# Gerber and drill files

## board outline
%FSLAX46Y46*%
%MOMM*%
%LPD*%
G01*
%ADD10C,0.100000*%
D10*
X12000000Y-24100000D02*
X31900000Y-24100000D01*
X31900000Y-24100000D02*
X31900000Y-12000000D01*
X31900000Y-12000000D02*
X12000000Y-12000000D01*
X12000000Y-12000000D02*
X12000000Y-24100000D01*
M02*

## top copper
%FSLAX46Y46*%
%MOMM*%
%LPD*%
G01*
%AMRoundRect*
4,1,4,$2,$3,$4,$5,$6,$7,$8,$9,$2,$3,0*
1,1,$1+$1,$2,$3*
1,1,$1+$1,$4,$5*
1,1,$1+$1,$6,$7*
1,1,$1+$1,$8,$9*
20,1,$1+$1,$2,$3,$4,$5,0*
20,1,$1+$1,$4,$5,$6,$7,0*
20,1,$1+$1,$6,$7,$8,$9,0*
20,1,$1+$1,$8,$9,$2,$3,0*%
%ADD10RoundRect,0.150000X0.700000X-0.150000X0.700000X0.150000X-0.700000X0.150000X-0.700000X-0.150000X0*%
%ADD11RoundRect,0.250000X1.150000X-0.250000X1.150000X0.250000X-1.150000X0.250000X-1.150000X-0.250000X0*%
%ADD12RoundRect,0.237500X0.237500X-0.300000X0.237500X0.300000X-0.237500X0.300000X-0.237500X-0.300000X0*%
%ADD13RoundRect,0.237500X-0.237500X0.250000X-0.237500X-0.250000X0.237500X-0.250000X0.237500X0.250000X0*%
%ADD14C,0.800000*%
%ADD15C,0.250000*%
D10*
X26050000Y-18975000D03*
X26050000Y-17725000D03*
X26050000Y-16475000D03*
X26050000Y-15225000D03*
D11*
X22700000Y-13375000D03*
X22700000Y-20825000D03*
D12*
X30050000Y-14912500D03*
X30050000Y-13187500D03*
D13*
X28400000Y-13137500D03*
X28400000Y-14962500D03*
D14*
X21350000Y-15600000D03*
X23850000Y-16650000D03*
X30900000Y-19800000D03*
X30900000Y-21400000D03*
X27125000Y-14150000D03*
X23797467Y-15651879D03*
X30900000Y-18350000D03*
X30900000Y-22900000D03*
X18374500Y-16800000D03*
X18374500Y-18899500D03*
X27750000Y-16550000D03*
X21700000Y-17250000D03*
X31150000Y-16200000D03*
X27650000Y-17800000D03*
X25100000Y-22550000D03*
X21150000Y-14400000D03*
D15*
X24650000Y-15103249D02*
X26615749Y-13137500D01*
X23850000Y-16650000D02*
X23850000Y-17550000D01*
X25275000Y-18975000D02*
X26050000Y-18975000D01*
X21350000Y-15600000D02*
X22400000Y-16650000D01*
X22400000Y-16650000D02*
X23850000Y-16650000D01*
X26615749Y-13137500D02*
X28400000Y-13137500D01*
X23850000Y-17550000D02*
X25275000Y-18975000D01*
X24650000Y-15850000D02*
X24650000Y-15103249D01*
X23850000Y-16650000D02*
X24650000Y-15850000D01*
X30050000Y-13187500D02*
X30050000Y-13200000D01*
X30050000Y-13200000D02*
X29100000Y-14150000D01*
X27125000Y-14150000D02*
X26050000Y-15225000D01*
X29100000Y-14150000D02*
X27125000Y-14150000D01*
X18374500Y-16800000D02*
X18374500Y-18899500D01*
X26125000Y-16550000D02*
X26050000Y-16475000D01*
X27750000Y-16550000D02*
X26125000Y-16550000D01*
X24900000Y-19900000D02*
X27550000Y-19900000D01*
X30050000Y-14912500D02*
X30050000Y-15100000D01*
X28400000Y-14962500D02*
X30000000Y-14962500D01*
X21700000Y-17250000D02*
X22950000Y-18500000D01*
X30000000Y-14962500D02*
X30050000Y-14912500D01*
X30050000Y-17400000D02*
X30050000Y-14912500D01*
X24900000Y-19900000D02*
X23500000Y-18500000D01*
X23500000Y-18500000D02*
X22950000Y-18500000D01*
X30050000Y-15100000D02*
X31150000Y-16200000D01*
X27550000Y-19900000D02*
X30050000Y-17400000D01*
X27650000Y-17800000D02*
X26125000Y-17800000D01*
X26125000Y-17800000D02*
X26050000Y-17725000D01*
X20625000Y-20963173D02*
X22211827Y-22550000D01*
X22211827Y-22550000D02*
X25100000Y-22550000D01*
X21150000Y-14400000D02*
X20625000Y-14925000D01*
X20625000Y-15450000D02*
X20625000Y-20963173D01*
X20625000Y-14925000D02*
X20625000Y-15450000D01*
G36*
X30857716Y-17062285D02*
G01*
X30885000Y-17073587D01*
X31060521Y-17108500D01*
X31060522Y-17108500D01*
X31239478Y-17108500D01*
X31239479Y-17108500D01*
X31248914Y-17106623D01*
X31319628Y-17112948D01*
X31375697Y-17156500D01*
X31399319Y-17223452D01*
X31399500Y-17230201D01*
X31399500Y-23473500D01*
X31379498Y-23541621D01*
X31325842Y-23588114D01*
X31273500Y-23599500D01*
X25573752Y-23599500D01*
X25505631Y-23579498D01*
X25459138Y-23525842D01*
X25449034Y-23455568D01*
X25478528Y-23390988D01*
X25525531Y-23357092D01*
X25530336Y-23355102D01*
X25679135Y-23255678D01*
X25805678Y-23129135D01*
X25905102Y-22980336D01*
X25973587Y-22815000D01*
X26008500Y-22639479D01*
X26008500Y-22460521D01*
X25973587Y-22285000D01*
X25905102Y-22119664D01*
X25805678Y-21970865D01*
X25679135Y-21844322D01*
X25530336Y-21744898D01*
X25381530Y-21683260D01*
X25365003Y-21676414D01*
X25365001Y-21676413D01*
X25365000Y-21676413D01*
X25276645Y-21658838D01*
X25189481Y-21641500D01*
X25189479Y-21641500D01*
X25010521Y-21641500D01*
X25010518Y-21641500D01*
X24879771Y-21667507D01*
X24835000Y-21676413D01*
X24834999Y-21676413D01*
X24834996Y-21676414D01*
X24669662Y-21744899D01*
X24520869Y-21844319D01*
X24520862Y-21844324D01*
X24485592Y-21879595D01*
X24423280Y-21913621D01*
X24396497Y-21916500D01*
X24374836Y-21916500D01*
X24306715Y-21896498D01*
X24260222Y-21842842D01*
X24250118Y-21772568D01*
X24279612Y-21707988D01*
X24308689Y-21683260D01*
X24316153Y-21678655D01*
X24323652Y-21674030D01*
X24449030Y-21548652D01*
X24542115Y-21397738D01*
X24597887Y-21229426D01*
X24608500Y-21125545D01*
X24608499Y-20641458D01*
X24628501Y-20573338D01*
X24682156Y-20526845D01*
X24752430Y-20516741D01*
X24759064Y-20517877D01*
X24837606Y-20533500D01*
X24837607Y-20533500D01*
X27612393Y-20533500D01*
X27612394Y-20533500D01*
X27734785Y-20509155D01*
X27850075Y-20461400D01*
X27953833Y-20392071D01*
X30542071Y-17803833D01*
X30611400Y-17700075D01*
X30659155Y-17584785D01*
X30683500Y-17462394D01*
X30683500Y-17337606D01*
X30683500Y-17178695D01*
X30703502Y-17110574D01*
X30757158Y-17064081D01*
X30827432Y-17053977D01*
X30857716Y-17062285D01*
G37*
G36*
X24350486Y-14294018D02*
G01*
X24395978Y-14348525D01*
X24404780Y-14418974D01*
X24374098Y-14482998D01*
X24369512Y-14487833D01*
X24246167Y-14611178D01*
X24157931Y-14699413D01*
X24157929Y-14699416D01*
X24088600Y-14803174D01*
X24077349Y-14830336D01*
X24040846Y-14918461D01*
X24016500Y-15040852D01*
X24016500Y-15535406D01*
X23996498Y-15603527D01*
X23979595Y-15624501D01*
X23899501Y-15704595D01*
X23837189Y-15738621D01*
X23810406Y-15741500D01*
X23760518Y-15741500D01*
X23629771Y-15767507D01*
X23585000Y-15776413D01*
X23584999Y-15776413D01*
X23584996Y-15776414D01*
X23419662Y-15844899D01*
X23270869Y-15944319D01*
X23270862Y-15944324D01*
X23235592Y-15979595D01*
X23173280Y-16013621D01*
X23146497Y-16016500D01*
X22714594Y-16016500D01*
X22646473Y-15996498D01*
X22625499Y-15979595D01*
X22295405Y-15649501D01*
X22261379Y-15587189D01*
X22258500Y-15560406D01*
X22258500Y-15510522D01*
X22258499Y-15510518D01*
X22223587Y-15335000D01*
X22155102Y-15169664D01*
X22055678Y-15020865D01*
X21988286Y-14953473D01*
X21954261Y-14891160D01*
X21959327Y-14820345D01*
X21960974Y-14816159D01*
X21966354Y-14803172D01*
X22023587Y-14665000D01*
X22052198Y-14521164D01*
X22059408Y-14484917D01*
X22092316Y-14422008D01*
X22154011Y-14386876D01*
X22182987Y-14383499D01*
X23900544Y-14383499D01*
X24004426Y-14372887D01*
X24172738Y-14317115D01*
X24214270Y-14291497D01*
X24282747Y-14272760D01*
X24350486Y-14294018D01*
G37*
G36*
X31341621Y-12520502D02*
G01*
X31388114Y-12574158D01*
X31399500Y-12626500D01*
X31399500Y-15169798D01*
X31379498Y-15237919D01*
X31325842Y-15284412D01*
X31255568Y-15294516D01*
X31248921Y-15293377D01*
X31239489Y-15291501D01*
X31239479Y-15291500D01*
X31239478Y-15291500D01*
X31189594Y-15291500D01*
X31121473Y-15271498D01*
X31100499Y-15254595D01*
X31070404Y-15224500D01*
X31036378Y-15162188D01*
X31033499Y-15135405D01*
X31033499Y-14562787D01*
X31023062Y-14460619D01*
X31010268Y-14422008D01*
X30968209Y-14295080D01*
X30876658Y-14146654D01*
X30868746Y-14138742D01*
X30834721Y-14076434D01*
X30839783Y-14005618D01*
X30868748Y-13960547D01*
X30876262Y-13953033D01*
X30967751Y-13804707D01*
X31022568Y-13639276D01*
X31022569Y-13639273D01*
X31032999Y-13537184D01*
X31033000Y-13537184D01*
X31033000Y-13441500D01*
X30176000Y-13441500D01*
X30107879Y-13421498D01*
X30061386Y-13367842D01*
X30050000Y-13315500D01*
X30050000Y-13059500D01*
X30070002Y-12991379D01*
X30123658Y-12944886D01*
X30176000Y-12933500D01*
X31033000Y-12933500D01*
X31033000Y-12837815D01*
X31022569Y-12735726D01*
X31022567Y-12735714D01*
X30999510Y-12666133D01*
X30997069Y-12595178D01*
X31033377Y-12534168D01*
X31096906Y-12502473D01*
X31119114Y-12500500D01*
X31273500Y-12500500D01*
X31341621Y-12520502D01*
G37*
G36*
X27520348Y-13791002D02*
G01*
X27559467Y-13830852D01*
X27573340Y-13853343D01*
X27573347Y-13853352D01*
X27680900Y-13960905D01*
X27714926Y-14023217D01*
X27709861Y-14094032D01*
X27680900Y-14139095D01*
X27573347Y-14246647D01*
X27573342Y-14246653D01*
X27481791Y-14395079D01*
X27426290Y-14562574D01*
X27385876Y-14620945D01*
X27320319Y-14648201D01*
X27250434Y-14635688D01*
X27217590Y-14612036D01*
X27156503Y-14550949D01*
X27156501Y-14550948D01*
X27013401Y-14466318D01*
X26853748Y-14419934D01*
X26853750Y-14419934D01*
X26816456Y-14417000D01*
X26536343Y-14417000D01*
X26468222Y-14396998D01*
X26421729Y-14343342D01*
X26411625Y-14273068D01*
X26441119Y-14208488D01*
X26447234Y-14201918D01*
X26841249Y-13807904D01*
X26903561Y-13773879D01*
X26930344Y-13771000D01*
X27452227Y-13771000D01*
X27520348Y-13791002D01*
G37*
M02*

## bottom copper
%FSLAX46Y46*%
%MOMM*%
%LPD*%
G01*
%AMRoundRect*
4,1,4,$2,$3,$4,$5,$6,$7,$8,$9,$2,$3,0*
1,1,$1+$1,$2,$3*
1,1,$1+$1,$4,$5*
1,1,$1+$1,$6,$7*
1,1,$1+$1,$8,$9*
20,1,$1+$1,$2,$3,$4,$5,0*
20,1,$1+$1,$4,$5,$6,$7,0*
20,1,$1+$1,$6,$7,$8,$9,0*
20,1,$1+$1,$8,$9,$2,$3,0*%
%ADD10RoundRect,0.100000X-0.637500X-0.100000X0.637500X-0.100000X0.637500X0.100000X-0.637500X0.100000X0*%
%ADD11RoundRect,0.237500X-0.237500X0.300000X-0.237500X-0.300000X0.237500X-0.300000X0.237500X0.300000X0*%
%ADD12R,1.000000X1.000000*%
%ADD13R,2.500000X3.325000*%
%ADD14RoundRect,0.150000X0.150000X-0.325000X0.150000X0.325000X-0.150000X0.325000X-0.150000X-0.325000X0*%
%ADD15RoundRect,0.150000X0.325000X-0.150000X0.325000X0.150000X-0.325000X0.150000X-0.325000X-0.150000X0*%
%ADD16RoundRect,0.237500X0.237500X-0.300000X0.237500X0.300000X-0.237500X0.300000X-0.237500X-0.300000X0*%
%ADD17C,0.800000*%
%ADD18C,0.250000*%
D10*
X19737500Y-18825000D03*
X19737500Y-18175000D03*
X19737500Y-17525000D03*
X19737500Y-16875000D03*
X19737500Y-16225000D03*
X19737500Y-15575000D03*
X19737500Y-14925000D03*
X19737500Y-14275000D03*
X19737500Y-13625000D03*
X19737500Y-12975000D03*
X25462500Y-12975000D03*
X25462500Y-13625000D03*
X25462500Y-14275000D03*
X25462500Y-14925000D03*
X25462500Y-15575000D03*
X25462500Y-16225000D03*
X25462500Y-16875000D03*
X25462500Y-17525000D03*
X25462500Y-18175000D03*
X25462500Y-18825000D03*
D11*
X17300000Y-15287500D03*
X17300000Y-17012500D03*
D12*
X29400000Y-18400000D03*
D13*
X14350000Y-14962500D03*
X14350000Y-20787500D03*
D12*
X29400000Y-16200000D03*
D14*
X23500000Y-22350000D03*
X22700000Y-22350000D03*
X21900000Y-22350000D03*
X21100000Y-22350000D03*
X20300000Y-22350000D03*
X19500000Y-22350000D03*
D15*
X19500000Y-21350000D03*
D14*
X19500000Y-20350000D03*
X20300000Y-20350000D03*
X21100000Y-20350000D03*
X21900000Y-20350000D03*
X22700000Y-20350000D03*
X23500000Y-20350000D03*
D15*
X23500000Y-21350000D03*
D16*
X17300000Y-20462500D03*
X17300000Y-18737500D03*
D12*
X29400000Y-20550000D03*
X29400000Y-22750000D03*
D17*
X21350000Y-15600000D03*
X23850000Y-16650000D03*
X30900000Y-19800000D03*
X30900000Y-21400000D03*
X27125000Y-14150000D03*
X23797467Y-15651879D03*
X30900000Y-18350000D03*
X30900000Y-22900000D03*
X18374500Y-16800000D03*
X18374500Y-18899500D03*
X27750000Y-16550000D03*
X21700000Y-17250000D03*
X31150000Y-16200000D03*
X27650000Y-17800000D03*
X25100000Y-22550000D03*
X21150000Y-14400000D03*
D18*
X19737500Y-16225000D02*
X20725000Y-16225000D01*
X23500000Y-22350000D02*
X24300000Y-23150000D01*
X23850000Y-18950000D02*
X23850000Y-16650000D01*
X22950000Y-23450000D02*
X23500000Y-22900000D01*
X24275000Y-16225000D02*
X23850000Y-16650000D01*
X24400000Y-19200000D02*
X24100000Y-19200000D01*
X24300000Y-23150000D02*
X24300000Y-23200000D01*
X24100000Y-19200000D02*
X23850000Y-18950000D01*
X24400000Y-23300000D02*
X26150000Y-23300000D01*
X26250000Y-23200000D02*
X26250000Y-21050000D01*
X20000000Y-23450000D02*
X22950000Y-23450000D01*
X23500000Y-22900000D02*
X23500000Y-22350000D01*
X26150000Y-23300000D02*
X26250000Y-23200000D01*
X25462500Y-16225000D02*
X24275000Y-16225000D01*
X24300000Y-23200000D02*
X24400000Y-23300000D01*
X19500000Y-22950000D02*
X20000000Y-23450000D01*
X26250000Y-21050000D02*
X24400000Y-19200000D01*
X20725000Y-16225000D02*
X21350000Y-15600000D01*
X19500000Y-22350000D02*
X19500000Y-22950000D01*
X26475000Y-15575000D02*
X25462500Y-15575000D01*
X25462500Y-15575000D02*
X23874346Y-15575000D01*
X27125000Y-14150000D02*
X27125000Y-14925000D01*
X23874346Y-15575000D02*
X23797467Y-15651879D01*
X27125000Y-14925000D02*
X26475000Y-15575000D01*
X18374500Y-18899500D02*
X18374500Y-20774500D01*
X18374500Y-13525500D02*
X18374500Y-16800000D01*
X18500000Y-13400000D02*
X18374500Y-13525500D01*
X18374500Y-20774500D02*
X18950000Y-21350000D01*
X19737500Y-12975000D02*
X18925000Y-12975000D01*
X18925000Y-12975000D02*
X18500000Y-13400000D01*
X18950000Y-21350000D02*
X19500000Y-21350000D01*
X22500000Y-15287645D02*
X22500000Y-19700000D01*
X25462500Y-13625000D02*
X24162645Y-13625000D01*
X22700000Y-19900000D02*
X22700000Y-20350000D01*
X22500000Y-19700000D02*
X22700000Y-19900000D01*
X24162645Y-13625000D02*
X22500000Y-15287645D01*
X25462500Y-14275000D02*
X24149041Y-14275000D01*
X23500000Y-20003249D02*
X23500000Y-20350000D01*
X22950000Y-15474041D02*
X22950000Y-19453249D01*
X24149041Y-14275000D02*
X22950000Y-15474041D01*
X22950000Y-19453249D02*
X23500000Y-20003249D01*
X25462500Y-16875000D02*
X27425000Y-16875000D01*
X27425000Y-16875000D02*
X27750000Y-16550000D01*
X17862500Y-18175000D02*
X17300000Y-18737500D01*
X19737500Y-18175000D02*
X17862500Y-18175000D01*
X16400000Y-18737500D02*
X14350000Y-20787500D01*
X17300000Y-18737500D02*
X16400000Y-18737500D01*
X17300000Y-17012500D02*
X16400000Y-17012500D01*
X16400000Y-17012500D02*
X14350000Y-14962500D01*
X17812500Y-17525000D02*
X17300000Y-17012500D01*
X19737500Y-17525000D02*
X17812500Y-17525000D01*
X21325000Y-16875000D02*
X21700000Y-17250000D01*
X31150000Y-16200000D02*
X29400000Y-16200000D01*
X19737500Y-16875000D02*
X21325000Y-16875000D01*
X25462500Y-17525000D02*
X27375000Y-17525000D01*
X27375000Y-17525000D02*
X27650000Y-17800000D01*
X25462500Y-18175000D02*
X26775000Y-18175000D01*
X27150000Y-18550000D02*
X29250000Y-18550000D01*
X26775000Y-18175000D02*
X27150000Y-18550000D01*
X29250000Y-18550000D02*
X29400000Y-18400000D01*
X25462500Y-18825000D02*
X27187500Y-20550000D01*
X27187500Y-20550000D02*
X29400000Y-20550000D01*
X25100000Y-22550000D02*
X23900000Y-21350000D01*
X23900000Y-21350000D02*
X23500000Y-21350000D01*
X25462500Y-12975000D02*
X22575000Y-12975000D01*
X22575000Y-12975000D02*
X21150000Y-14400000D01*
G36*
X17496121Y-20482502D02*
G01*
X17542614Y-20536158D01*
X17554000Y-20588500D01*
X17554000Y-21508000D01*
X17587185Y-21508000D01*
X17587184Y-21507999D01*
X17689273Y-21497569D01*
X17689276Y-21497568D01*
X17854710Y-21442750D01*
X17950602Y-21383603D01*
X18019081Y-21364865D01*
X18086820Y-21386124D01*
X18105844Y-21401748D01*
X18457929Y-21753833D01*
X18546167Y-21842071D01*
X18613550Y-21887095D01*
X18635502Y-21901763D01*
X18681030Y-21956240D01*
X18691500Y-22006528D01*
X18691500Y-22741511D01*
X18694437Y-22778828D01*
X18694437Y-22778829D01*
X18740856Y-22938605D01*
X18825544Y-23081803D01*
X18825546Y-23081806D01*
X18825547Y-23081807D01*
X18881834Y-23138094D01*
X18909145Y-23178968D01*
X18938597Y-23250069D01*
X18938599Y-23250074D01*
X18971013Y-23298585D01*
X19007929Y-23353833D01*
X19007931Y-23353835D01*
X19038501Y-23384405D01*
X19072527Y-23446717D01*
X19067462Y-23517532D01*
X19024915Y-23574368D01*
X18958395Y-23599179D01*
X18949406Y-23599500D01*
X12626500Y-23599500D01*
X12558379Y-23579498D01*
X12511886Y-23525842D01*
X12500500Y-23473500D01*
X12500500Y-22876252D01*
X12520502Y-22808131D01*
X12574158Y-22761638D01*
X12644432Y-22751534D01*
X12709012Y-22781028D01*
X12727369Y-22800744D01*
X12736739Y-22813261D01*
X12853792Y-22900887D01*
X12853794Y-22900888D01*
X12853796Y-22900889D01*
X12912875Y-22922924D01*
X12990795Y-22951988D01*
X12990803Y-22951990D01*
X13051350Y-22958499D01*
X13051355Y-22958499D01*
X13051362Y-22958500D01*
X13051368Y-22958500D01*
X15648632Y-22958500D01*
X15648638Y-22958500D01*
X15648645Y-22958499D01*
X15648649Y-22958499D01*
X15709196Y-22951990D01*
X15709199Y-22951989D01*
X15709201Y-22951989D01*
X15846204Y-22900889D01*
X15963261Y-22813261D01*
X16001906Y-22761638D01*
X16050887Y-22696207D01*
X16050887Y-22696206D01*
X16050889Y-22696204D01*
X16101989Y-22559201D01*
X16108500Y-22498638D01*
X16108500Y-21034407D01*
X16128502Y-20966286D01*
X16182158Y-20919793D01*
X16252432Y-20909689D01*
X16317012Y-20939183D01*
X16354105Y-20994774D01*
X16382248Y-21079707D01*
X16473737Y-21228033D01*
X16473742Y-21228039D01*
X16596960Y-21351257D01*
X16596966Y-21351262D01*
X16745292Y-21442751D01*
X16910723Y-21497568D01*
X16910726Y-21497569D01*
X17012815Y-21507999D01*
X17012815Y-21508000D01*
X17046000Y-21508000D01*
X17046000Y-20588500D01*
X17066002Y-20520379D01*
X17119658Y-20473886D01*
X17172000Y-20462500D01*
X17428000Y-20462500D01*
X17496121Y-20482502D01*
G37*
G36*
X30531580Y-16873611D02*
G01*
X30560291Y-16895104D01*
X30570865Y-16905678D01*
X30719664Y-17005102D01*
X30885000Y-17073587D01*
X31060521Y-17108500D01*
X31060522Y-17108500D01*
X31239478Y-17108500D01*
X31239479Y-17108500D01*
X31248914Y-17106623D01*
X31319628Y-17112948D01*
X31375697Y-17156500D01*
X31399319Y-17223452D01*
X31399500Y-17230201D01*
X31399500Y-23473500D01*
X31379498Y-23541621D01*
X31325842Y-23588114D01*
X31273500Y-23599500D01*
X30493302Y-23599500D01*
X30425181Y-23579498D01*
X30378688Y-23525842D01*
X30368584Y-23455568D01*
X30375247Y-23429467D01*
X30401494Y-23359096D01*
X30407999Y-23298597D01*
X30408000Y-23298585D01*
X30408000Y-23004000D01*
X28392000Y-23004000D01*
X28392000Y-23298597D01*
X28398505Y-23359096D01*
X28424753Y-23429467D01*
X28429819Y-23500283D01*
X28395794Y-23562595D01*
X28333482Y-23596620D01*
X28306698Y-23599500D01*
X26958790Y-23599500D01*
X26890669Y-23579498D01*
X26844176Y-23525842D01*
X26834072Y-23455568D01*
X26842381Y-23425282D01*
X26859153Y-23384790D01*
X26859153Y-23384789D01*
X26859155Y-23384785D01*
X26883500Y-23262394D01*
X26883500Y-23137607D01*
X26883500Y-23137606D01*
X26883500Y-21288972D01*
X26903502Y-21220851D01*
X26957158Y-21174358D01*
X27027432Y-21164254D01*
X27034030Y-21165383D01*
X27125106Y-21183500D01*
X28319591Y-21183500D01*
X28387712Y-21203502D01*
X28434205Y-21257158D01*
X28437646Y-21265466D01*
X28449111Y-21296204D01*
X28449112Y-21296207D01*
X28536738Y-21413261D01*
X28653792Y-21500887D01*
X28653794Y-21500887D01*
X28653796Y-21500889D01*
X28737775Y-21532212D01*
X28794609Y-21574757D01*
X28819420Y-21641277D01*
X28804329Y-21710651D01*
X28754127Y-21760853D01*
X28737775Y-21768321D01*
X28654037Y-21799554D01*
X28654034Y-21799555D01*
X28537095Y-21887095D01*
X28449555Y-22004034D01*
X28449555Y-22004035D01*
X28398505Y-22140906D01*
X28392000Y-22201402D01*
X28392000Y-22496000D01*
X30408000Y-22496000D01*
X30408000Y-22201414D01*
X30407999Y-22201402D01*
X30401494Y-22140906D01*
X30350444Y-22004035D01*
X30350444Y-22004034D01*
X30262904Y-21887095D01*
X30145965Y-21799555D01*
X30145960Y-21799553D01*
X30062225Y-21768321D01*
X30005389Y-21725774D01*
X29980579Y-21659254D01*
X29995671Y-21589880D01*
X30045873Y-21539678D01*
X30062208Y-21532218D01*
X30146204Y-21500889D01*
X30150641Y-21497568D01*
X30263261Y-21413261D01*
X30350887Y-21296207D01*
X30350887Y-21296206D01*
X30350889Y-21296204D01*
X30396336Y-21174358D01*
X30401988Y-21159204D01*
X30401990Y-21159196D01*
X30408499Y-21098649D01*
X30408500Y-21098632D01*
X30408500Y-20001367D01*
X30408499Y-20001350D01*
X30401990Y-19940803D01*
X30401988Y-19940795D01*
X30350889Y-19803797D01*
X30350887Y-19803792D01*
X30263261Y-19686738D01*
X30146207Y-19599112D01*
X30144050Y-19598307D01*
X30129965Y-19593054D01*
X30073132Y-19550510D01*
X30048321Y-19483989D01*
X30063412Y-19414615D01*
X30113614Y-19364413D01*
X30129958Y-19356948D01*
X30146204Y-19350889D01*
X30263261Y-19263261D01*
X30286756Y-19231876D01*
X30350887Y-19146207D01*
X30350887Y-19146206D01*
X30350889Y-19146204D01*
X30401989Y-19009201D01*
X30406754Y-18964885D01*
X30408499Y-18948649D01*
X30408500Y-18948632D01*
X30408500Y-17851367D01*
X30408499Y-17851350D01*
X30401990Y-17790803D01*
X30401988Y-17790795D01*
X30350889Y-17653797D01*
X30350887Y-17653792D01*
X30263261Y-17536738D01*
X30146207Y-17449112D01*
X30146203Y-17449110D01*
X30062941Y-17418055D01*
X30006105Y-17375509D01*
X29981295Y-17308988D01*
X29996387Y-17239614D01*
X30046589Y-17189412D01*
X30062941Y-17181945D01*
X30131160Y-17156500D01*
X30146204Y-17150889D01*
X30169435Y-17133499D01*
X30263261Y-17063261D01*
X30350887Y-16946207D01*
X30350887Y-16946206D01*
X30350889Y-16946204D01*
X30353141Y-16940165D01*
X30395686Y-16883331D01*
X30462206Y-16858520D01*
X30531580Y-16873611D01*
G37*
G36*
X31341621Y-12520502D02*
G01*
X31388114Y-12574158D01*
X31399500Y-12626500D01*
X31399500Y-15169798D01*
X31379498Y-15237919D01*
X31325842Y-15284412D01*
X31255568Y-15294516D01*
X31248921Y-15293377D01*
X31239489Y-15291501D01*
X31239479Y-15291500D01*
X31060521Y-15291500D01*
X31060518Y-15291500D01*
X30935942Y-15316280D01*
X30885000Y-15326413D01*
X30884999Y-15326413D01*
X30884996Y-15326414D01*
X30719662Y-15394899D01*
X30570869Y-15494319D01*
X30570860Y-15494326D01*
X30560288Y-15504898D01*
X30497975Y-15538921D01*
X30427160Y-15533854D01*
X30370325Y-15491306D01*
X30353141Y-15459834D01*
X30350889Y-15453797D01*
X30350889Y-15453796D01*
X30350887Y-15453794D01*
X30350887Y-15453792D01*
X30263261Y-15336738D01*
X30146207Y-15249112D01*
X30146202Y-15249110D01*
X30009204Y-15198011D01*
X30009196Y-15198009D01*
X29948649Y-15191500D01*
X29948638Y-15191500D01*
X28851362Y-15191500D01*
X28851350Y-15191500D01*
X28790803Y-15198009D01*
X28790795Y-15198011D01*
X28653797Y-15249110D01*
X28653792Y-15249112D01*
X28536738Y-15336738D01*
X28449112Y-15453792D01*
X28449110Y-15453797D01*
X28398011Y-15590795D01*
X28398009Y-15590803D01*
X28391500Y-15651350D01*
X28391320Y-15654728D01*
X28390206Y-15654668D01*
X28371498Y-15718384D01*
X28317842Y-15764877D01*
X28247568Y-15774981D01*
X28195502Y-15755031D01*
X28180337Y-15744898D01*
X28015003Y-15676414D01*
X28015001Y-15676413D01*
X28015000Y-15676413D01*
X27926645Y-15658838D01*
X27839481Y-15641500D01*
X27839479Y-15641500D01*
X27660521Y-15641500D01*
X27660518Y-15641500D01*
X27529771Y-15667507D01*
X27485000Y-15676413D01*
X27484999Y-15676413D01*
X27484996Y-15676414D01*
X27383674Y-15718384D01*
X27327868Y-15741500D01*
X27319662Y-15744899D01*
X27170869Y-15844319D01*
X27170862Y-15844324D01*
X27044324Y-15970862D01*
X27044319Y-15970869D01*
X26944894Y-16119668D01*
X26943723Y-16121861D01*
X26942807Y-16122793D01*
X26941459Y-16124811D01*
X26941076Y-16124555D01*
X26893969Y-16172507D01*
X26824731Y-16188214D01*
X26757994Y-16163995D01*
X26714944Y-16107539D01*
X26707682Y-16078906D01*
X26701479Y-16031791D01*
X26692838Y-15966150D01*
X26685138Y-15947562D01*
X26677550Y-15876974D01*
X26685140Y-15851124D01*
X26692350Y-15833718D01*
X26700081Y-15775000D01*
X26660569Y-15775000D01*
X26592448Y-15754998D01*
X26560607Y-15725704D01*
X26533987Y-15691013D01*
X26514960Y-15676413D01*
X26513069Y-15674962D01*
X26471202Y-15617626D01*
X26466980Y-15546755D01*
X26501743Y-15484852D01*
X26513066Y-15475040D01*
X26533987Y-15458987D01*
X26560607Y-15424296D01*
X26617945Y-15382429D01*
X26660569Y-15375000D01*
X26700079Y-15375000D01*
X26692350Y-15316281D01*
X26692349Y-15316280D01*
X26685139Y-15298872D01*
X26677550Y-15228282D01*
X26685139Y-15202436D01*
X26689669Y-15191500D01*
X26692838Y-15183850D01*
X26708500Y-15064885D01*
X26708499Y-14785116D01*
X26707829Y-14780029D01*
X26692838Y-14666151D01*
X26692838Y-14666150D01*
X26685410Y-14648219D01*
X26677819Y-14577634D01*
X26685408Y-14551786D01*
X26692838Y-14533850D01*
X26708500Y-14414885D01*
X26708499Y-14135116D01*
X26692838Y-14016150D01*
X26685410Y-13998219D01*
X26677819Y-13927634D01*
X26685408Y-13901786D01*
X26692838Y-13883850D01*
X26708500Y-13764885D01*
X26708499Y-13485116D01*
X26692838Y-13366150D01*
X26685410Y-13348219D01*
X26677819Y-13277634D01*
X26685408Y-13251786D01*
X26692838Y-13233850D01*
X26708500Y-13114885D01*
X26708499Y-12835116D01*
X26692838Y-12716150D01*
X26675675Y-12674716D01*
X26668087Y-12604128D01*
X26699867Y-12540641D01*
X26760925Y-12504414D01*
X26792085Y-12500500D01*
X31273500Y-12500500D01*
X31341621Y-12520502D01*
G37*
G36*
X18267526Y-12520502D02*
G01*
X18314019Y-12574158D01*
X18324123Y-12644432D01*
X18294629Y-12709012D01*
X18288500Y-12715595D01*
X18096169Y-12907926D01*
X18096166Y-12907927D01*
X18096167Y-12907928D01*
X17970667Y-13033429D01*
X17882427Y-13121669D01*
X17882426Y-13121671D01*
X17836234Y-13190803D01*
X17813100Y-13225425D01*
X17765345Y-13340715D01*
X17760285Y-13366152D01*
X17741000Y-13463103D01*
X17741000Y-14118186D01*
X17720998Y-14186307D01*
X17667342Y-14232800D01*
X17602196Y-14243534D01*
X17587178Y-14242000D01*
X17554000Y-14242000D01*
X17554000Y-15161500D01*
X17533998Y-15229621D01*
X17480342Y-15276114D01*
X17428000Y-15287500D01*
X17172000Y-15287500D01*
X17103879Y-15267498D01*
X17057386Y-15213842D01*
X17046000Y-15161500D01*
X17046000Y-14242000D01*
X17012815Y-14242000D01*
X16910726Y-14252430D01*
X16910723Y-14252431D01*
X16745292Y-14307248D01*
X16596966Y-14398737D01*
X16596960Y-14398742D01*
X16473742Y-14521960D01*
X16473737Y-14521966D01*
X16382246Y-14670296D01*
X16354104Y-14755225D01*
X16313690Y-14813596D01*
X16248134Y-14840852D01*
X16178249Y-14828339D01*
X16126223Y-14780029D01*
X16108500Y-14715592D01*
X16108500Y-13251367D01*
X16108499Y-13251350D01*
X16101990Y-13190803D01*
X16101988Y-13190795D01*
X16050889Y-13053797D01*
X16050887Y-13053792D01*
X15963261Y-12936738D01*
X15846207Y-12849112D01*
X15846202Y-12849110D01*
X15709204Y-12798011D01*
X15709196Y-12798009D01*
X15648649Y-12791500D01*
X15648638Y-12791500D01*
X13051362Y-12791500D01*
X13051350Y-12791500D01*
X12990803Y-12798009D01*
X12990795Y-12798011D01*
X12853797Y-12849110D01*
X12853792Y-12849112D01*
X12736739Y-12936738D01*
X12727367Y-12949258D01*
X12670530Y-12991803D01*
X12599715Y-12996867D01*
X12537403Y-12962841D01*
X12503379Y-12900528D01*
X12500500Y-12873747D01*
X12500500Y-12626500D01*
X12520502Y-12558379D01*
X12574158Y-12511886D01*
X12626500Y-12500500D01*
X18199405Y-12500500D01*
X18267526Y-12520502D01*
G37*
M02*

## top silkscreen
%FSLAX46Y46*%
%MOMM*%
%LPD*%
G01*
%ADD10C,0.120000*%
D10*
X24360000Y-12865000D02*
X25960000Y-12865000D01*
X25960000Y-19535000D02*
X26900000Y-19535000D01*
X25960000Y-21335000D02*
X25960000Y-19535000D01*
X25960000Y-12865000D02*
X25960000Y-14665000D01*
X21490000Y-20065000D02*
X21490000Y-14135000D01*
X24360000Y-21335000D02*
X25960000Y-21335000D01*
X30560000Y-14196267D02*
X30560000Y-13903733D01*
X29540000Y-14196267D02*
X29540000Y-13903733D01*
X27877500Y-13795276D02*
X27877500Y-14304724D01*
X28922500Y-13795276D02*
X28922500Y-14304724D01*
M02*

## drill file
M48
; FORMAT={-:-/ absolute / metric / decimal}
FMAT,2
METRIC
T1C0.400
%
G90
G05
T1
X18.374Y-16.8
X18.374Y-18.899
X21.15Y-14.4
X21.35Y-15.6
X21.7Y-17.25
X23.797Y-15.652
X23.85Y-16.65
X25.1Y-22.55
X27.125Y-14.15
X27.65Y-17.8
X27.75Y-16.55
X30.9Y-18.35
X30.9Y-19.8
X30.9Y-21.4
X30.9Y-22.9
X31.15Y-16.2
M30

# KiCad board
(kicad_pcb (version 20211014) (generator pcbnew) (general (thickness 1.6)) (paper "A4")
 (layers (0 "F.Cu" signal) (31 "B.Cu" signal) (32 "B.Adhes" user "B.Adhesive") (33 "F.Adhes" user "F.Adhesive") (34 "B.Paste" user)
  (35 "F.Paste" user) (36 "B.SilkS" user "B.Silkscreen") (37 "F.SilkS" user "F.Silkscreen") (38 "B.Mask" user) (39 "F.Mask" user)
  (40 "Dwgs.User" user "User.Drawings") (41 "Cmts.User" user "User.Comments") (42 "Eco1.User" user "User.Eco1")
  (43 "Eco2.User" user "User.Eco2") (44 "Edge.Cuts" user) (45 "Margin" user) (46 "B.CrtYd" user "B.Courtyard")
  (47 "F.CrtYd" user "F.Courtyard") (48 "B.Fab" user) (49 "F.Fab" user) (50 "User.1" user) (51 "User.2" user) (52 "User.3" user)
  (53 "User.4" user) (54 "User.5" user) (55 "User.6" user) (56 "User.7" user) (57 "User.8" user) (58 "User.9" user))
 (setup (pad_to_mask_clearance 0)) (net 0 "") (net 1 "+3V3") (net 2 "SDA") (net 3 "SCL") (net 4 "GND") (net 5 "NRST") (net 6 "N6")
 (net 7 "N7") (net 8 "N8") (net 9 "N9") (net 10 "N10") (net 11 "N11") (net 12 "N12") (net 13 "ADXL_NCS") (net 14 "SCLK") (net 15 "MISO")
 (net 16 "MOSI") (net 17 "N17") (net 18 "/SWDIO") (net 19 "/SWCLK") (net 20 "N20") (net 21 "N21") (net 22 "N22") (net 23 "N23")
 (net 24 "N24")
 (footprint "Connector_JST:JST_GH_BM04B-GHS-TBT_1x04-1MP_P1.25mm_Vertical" (layer "F.Cu") (at 24.1 17.1 90)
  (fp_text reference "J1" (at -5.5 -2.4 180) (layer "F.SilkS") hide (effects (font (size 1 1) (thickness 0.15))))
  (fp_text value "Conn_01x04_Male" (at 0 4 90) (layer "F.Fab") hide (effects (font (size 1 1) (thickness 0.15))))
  (fp_line (start 4.235 0.26) (end 4.235 1.86) (layer "F.SilkS") (width 0.12))
  (fp_line (start -2.435 1.86) (end -2.435 2.8) (layer "F.SilkS") (width 0.12))
  (fp_line (start -4.235 1.86) (end -2.435 1.86) (layer "F.SilkS") (width 0.12))
  (fp_line (start 4.235 1.86) (end 2.435 1.86) (layer "F.SilkS") (width 0.12))
  (fp_line (start -2.965 -2.61) (end 2.965 -2.61) (layer "F.SilkS") (width 0.12))
  (fp_line (start -4.235 0.26) (end -4.235 1.86) (layer "F.SilkS") (width 0.12))
  (pad "1" smd roundrect (at -1.875 1.95 90) (size 0.6 1.7) (layers "F.Cu" "F.Paste" "F.Mask") (roundrect_rratio 0.25) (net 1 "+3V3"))
  (pad "2" smd roundrect (at -0.625 1.95 90) (size 0.6 1.7) (layers "F.Cu" "F.Paste" "F.Mask") (roundrect_rratio 0.25) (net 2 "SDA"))
  (pad "3" smd roundrect (at 0.625 1.95 90) (size 0.6 1.7) (layers "F.Cu" "F.Paste" "F.Mask") (roundrect_rratio 0.25) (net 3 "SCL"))
  (pad "4" smd roundrect (at 1.875 1.95 90) (size 0.6 1.7) (layers "F.Cu" "F.Paste" "F.Mask") (roundrect_rratio 0.25) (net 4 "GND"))
  (pad "MP" smd roundrect (at 3.725 -1.4 90) (size 1 2.8) (layers "F.Cu" "F.Paste" "F.Mask") (roundrect_rratio 0.25))
  (pad "MP" smd roundrect (at -3.725 -1.4 90) (size 1 2.8) (layers "F.Cu" "F.Paste" "F.Mask") (roundrect_rratio 0.25)))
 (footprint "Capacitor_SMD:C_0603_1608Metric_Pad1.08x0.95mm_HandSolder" (layer "F.Cu") (at 30.05 14.05 90)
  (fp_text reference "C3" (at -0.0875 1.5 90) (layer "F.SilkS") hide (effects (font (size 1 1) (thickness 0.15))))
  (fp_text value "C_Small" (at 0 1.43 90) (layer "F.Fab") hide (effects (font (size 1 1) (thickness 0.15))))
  (fp_line (start -0.146267 0.51) (end 0.146267 0.51) (layer "F.SilkS") (width 0.12))
  (fp_line (start -0.146267 -0.51) (end 0.146267 -0.51) (layer "F.SilkS") (width 0.12))
  (pad "1" smd roundrect (at -0.8625 0 90) (size 1.075 0.95) (layers "F.Cu" "F.Paste" "F.Mask") (roundrect_rratio 0.25) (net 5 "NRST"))
  (pad "2" smd roundrect (at 0.8625 0 90) (size 1.075 0.95) (layers "F.Cu" "F.Paste" "F.Mask") (roundrect_rratio 0.25) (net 4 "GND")))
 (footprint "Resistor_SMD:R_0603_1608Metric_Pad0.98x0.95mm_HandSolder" (layer "F.Cu") (at 28.4 14.05 -90)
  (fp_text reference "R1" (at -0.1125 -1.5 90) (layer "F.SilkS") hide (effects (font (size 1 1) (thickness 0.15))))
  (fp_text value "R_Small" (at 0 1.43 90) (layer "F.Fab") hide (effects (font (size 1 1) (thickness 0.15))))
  (fp_line (start -0.254724 0.5225) (end 0.254724 0.5225) (layer "F.SilkS") (width 0.12))
  (fp_line (start -0.254724 -0.5225) (end 0.254724 -0.5225) (layer "F.SilkS") (width 0.12))
  (pad "1" smd roundrect (at -0.9125 0 270) (size 0.975 0.95) (layers "F.Cu" "F.Paste" "F.Mask") (roundrect_rratio 0.25) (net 1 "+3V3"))
  (pad "2" smd roundrect (at 0.9125 0 270) (size 0.975 0.95) (layers "F.Cu" "F.Paste" "F.Mask") (roundrect_rratio 0.25) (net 5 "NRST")))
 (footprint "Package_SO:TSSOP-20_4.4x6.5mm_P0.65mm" (layer "B.Cu") (at 22.6 15.9)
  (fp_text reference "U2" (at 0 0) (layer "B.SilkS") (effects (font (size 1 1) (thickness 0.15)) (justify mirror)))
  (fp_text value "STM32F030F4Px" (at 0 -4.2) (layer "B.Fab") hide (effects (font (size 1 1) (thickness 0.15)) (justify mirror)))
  (pad "1" smd roundrect (at -2.8625 2.925) (size 1.475 0.4) (layers "B.Cu" "B.Paste" "B.Mask") (roundrect_rratio 0.25) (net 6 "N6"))
  (pad "2" smd roundrect (at -2.8625 2.275) (size 1.475 0.4) (layers "B.Cu" "B.Paste" "B.Mask") (roundrect_rratio 0.25) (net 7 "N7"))
  (pad "3" smd roundrect (at -2.8625 1.625) (size 1.475 0.4) (layers "B.Cu" "B.Paste" "B.Mask") (roundrect_rratio 0.25) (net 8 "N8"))
  (pad "4" smd roundrect (at -2.8625 0.975) (size 1.475 0.4) (layers "B.Cu" "B.Paste" "B.Mask") (roundrect_rratio 0.25) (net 5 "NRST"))
  (pad "5" smd roundrect (at -2.8625 0.325) (size 1.475 0.4) (layers "B.Cu" "B.Paste" "B.Mask") (roundrect_rratio 0.25) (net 1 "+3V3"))
  (pad "6" smd roundrect (at -2.8625 -0.325) (size 1.475 0.4) (layers "B.Cu" "B.Paste" "B.Mask") (roundrect_rratio 0.25) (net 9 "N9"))
  (pad "7" smd roundrect (at -2.8625 -0.975) (size 1.475 0.4) (layers "B.Cu" "B.Paste" "B.Mask") (roundrect_rratio 0.25) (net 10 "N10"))
  (pad "8" smd roundrect (at -2.8625 -1.625) (size 1.475 0.4) (layers "B.Cu" "B.Paste" "B.Mask") (roundrect_rratio 0.25) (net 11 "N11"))
  (pad "9" smd roundrect (at -2.8625 -2.275) (size 1.475 0.4) (layers "B.Cu" "B.Paste" "B.Mask") (roundrect_rratio 0.25) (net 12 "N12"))
  (pad "10" smd roundrect (at -2.8625 -2.925) (size 1.475 0.4) (layers "B.Cu" "B.Paste" "B.Mask") (roundrect_rratio 0.25)
   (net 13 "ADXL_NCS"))
  (pad "11" smd roundrect (at 2.8625 -2.925) (size 1.475 0.4) (layers "B.Cu" "B.Paste" "B.Mask") (roundrect_rratio 0.25) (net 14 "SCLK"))
  (pad "12" smd roundrect (at 2.8625 -2.275) (size 1.475 0.4) (layers "B.Cu" "B.Paste" "B.Mask") (roundrect_rratio 0.25) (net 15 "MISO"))
  (pad "13" smd roundrect (at 2.8625 -1.625) (size 1.475 0.4) (layers "B.Cu" "B.Paste" "B.Mask") (roundrect_rratio 0.25) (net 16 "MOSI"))
  (pad "14" smd roundrect (at 2.8625 -0.975) (size 1.475 0.4) (layers "B.Cu" "B.Paste" "B.Mask") (roundrect_rratio 0.25) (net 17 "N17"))
  (pad "15" smd roundrect (at 2.8625 -0.325) (size 1.475 0.4) (layers "B.Cu" "B.Paste" "B.Mask") (roundrect_rratio 0.25) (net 4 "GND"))
  (pad "16" smd roundrect (at 2.8625 0.325) (size 1.475 0.4) (layers "B.Cu" "B.Paste" "B.Mask") (roundrect_rratio 0.25) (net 1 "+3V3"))
  (pad "17" smd roundrect (at 2.8625 0.975) (size 1.475 0.4) (layers "B.Cu" "B.Paste" "B.Mask") (roundrect_rratio 0.25) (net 3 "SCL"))
  (pad "18" smd roundrect (at 2.8625 1.625) (size 1.475 0.4) (layers "B.Cu" "B.Paste" "B.Mask") (roundrect_rratio 0.25) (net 2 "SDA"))
  (pad "19" smd roundrect (at 2.8625 2.275) (size 1.475 0.4) (layers "B.Cu" "B.Paste" "B.Mask") (roundrect_rratio 0.25) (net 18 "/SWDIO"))
  (pad "20" smd roundrect (at 2.8625 2.925) (size 1.475 0.4) (layers "B.Cu" "B.Paste" "B.Mask") (roundrect_rratio 0.25) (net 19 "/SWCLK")))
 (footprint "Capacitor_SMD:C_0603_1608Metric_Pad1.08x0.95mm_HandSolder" (layer "B.Cu") (at 17.3 16.15 -90)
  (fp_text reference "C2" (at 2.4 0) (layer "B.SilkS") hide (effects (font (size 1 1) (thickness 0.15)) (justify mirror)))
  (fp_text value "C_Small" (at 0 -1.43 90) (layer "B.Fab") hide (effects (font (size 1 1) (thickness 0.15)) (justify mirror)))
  (pad "1" smd roundrect (at -0.8625 0 270) (size 1.075 0.95) (layers "B.Cu" "B.Paste" "B.Mask") (roundrect_rratio 0.25) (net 4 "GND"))
  (pad "2" smd roundrect (at 0.8625 0 270) (size 1.075 0.95) (layers "B.Cu" "B.Paste" "B.Mask") (roundrect_rratio 0.25) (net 8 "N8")))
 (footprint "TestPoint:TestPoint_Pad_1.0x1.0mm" (layer "B.Cu") (at 29.4 18.4 180)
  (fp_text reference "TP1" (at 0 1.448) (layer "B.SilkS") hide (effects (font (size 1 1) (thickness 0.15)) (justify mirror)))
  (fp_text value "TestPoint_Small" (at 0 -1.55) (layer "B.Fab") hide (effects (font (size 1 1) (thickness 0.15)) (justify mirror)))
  (pad "1" smd rect (at 0 0 180) (size 1 1) (layers "B.Cu" "B.Mask") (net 18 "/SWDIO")))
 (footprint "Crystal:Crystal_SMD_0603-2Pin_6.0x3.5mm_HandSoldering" (layer "B.Cu") (at 14.35 17.875 -90)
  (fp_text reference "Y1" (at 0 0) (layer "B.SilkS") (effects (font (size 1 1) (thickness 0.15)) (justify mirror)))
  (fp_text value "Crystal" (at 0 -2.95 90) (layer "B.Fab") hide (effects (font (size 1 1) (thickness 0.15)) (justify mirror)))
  (pad "1" smd rect (at -2.9125 0 270) (size 3.325 2.5) (layers "B.Cu" "B.Paste" "B.Mask") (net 8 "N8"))
  (pad "2" smd rect (at 2.9125 0 270) (size 3.325 2.5) (layers "B.Cu" "B.Paste" "B.Mask") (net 7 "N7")))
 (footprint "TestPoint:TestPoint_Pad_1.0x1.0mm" (layer "B.Cu") (at 29.4 16.2 180)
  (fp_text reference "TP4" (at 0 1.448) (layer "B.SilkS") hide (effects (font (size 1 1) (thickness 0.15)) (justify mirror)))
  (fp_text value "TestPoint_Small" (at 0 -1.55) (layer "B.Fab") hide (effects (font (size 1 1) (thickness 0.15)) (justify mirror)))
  (pad "1" smd rect (at 0 0 180) (size 1 1) (layers "B.Cu" "B.Mask") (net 5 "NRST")))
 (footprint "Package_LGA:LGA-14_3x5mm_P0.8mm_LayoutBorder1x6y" (layer "B.Cu") (at 21.5 21.35 90)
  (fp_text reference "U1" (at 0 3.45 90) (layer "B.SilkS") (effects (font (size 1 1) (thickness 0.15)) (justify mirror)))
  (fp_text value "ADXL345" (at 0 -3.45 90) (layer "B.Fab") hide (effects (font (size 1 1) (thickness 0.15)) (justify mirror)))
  (pad "1" smd roundrect (at -1 2 90) (size 0.95 0.6) (layers "B.Cu" "B.Paste" "B.Mask") (roundrect_rratio 0.25) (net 1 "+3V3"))
  (pad "2" smd roundrect (at -1 1.2 90) (size 0.95 0.6) (layers "B.Cu" "B.Paste" "B.Mask") (roundrect_rratio 0.25) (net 4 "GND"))
  (pad "3" smd roundrect (at -1 0.4 90) (size 0.95 0.6) (layers "B.Cu" "B.Paste" "B.Mask") (roundrect_rratio 0.25) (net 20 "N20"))
  (pad "4" smd roundrect (at -1 -0.4 90) (size 0.95 0.6) (layers "B.Cu" "B.Paste" "B.Mask") (roundrect_rratio 0.25) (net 4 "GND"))
  (pad "5" smd roundrect (at -1 -1.2 90) (size 0.95 0.6) (layers "B.Cu" "B.Paste" "B.Mask") (roundrect_rratio 0.25) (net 4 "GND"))
  (pad "6" smd roundrect (at -1 -2 90) (size 0.95 0.6) (layers "B.Cu" "B.Paste" "B.Mask") (roundrect_rratio 0.25) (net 1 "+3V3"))
  (pad "7" smd roundrect (at 0 -2 90) (size 0.6 0.95) (layers "B.Cu" "B.Paste" "B.Mask") (roundrect_rratio 0.25) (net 13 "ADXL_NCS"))
  (pad "8" smd roundrect (at 1 -2 90) (size 0.95 0.6) (layers "B.Cu" "B.Paste" "B.Mask") (roundrect_rratio 0.25) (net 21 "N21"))
  (pad "9" smd roundrect (at 1 -1.2 90) (size 0.95 0.6) (layers "B.Cu" "B.Paste" "B.Mask") (roundrect_rratio 0.25) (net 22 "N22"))
  (pad "10" smd roundrect (at 1 -0.4 90) (size 0.95 0.6) (layers "B.Cu" "B.Paste" "B.Mask") (roundrect_rratio 0.25) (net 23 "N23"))
  (pad "11" smd roundrect (at 1 0.4 90) (size 0.95 0.6) (layers "B.Cu" "B.Paste" "B.Mask") (roundrect_rratio 0.25) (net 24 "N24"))
  (pad "12" smd roundrect (at 1 1.2 90) (size 0.95 0.6) (layers "B.Cu" "B.Paste" "B.Mask") (roundrect_rratio 0.25) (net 15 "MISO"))
  (pad "13" smd roundrect (at 1 2 90) (size 0.95 0.6) (layers "B.Cu" "B.Paste" "B.Mask") (roundrect_rratio 0.25) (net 16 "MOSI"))
  (pad "14" smd roundrect (at 0 2 90) (size 0.6 0.95) (layers "B.Cu" "B.Paste" "B.Mask") (roundrect_rratio 0.25) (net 14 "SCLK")))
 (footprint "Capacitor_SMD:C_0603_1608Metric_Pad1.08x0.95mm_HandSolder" (layer "B.Cu") (at 17.3 19.6 90)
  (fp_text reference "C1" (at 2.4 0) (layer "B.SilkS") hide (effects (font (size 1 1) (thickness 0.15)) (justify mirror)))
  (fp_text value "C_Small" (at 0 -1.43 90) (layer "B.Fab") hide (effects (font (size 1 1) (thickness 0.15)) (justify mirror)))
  (pad "1" smd roundrect (at -0.8625 0 90) (size 1.075 0.95) (layers "B.Cu" "B.Paste" "B.Mask") (roundrect_rratio 0.25) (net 4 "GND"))
  (pad "2" smd roundrect (at 0.8625 0 90) (size 1.075 0.95) (layers "B.Cu" "B.Paste" "B.Mask") (roundrect_rratio 0.25) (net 7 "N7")))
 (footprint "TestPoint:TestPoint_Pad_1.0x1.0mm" (layer "B.Cu") (at 29.4 20.55 180)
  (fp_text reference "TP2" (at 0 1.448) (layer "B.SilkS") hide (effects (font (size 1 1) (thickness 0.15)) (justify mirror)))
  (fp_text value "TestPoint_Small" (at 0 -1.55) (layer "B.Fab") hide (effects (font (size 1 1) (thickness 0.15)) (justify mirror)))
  (pad "1" smd rect (at 0 0 180) (size 1 1) (layers "B.Cu" "B.Mask") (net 19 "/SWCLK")))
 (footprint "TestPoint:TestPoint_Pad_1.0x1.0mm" (layer "B.Cu") (at 29.4 22.75 180)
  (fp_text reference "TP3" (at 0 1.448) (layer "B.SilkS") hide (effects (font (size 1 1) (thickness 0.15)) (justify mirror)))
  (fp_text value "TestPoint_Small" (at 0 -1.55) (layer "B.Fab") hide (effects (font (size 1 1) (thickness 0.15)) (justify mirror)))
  (pad "1" smd rect (at 0 0 180) (size 1 1) (layers "B.Cu" "B.Mask") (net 4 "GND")))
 (gr_line (start 12 24.1) (end 31.9 24.1) (layer "Edge.Cuts") (width 0.1))
 (gr_line (start 31.9 24.1) (end 31.9 12) (layer "Edge.Cuts") (width 0.1))
 (gr_line (start 31.9 12) (end 12 12) (layer "Edge.Cuts") (width 0.1))
 (gr_line (start 12 12) (end 12 24.1) (layer "Edge.Cuts") (width 0.1))
 (segment (start 24.65 15.103249) (end 26.615749 13.1375) (width 0.25) (layer "F.Cu") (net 1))
 (segment (start 23.85 16.65) (end 23.85 17.55) (width 0.25) (layer "F.Cu") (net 1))
 (segment (start 25.275 18.975) (end 26.05 18.975) (width 0.25) (layer "F.Cu") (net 1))
 (segment (start 21.35 15.6) (end 22.4 16.65) (width 0.25) (layer "F.Cu") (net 1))
 (segment (start 22.4 16.65) (end 23.85 16.65) (width 0.25) (layer "F.Cu") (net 1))
 (segment (start 26.615749 13.1375) (end 28.4 13.1375) (width 0.25) (layer "F.Cu") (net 1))
 (segment (start 23.85 17.55) (end 25.275 18.975) (width 0.25) (layer "F.Cu") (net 1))
 (segment (start 24.65 15.85) (end 24.65 15.103249) (width 0.25) (layer "F.Cu") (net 1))
 (segment (start 23.85 16.65) (end 24.65 15.85) (width 0.25) (layer "F.Cu") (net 1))
 (via (at 21.35 15.6) (size 0.8) (drill 0.4) (layers "F.Cu" "B.Cu") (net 1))
 (via (at 23.85 16.65) (size 0.8) (drill 0.4) (layers "F.Cu" "B.Cu") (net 1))
 (segment (start 19.7375 16.225) (end 20.725 16.225) (width 0.25) (layer "B.Cu") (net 1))
 (segment (start 23.5 22.35) (end 24.3 23.15) (width 0.25) (layer "B.Cu") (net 1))
 (segment (start 23.85 18.95) (end 23.85 16.65) (width 0.25) (layer "B.Cu") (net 1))
 (segment (start 22.95 23.45) (end 23.5 22.9) (width 0.25) (layer "B.Cu") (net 1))
 (segment (start 24.275 16.225) (end 23.85 16.65) (width 0.25) (layer "B.Cu") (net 1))
 (segment (start 24.4 19.2) (end 24.1 19.2) (width 0.25) (layer "B.Cu") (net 1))
 (segment (start 24.3 23.15) (end 24.3 23.2) (width 0.25) (layer "B.Cu") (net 1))
 (segment (start 24.1 19.2) (end 23.85 18.95) (width 0.25) (layer "B.Cu") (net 1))
 (segment (start 24.4 23.3) (end 26.15 23.3) (width 0.25) (layer "B.Cu") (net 1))
 (segment (start 26.25 23.2) (end 26.25 21.05) (width 0.25) (layer "B.Cu") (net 1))
 (segment (start 20 23.45) (end 22.95 23.45) (width 0.25) (layer "B.Cu") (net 1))
 (segment (start 23.5 22.9) (end 23.5 22.35) (width 0.25) (layer "B.Cu") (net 1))
 (segment (start 26.15 23.3) (end 26.25 23.2) (width 0.25) (layer "B.Cu") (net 1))
 (segment (start 25.4625 16.225) (end 24.275 16.225) (width 0.25) (layer "B.Cu") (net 1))
 (segment (start 24.3 23.2) (end 24.4 23.3) (width 0.25) (layer "B.Cu") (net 1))
 (segment (start 19.5 22.95) (end 20 23.45) (width 0.25) (layer "B.Cu") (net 1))
 (segment (start 26.25 21.05) (end 24.4 19.2) (width 0.25) (layer "B.Cu") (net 1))
 (segment (start 20.725 16.225) (end 21.35 15.6) (width 0.25) (layer "B.Cu") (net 1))
 (segment (start 19.5 22.35) (end 19.5 22.95) (width 0.25) (layer "B.Cu") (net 1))
 (segment (start 30.05 13.1875) (end 30.05 13.2) (width 0.25) (layer "F.Cu") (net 4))
 (segment (start 30.05 13.2) (end 29.1 14.15) (width 0.25) (layer "F.Cu") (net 4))
 (segment (start 27.125 14.15) (end 26.05 15.225) (width 0.25) (layer "F.Cu") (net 4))
 (segment (start 29.1 14.15) (end 27.125 14.15) (width 0.25) (layer "F.Cu") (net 4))
 (via (at 30.9 19.8) (size 0.8) (drill 0.4) (layers "F.Cu" "B.Cu") (free) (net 4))
 (via (at 30.9 21.4) (size 0.8) (drill 0.4) (layers "F.Cu" "B.Cu") (free) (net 4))
 (via (at 27.125 14.15) (size 0.8) (drill 0.4) (layers "F.Cu" "B.Cu") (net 4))
 (via (at 23.797467 15.651879) (size 0.8) (drill 0.4) (layers "F.Cu" "B.Cu") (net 4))
 (via (at 30.9 18.35) (size 0.8) (drill 0.4) (layers "F.Cu" "B.Cu") (free) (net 4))
 (via (at 30.9 22.9) (size 0.8) (drill 0.4) (layers "F.Cu" "B.Cu") (free) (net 4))
 (segment (start 26.475 15.575) (end 25.4625 15.575) (width 0.25) (layer "B.Cu") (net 4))
 (segment (start 25.4625 15.575) (end 23.874346 15.575) (width 0.25) (layer "B.Cu") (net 4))
 (segment (start 27.125 14.15) (end 27.125 14.925) (width 0.25) (layer "B.Cu") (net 4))
 (segment (start 23.874346 15.575) (end 23.797467 15.651879) (width 0.25) (layer "B.Cu") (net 4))
 (segment (start 27.125 14.925) (end 26.475 15.575) (width 0.25) (layer "B.Cu") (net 4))
 (segment (start 18.3745 16.8) (end 18.3745 18.8995) (width 0.25) (layer "F.Cu") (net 13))
 (via (at 18.3745 16.8) (size 0.8) (drill 0.4) (layers "F.Cu" "B.Cu") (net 13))
 (via (at 18.3745 18.8995) (size 0.8) (drill 0.4) (layers "F.Cu" "B.Cu") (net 13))
 (segment (start 18.3745 18.8995) (end 18.3745 20.7745) (width 0.25) (layer "B.Cu") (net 13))
 (segment (start 18.3745 13.5255) (end 18.3745 16.8) (width 0.25) (layer "B.Cu") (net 13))
 (segment (start 18.5 13.4) (end 18.3745 13.5255) (width 0.25) (layer "B.Cu") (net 13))
 (segment (start 18.3745 20.7745) (end 18.95 21.35) (width 0.25) (layer "B.Cu") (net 13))
 (segment (start 19.7375 12.975) (end 18.925 12.975) (width 0.25) (layer "B.Cu") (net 13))
 (segment (start 18.925 12.975) (end 18.5 13.4) (width 0.25) (layer "B.Cu") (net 13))
 (segment (start 18.95 21.35) (end 19.5 21.35) (width 0.25) (layer "B.Cu") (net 13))
 (segment (start 22.5 15.287645) (end 22.5 19.7) (width 0.25) (layer "B.Cu") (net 15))
 (segment (start 25.4625 13.625) (end 24.162645 13.625) (width 0.25) (layer "B.Cu") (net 15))
 (segment (start 22.7 19.9) (end 22.7 20.35) (width 0.25) (layer "B.Cu") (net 15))
 (segment (start 22.5 19.7) (end 22.7 19.9) (width 0.25) (layer "B.Cu") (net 15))
 (segment (start 24.162645 13.625) (end 22.5 15.287645) (width 0.25) (layer "B.Cu") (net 15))
 (segment (start 25.4625 14.275) (end 24.149041 14.275) (width 0.25) (layer "B.Cu") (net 16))
 (segment (start 23.5 20.003249) (end 23.5 20.35) (width 0.25) (layer "B.Cu") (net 16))
 (segment (start 22.95 15.474041) (end 22.95 19.453249) (width 0.25) (layer "B.Cu") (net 16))
 (segment (start 24.149041 14.275) (end 22.95 15.474041) (width 0.25) (layer "B.Cu") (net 16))
 (segment (start 22.95 19.453249) (end 23.5 20.003249) (width 0.25) (layer "B.Cu") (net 16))
 (segment (start 26.125 16.55) (end 26.05 16.475) (width 0.25) (layer "F.Cu") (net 3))
 (segment (start 27.75 16.55) (end 26.125 16.55) (width 0.25) (layer "F.Cu") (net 3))
 (via (at 27.75 16.55) (size 0.8) (drill 0.4) (layers "F.Cu" "B.Cu") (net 3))
 (segment (start 25.4625 16.875) (end 27.425 16.875) (width 0.25) (layer "B.Cu") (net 3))
 (segment (start 27.425 16.875) (end 27.75 16.55) (width 0.25) (layer "B.Cu") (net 3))
 (segment (start 17.8625 18.175) (end 17.3 18.7375) (width 0.25) (layer "B.Cu") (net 7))
 (segment (start 19.7375 18.175) (end 17.8625 18.175) (width 0.25) (layer "B.Cu") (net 7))
 (segment (start 16.4 18.7375) (end 14.35 20.7875) (width 0.25) (layer "B.Cu") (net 7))
 (segment (start 17.3 18.7375) (end 16.4 18.7375) (width 0.25) (layer "B.Cu") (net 7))
 (segment (start 17.3 17.0125) (end 16.4 17.0125) (width 0.25) (layer "B.Cu") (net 8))
 (segment (start 16.4 17.0125) (end 14.35 14.9625) (width 0.25) (layer "B.Cu") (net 8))
 (segment (start 17.8125 17.525) (end 17.3 17.0125) (width 0.25) (layer "B.Cu") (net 8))
 (segment (start 19.7375 17.525) (end 17.8125 17.525) (width 0.25) (layer "B.Cu") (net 8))
 (segment (start 24.9 19.9) (end 27.55 19.9) (width 0.25) (layer "F.Cu") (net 5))
 (segment (start 30.05 14.9125) (end 30.05 15.1) (width 0.25) (layer "F.Cu") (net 5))
 (segment (start 28.4 14.9625) (end 30 14.9625) (width 0.25) (layer "F.Cu") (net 5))
 (segment (start 21.7 17.25) (end 22.95 18.5) (width 0.25) (layer "F.Cu") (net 5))
 (segment (start 30 14.9625) (end 30.05 14.9125) (width 0.25) (layer "F.Cu") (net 5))
 (segment (start 30.05 17.4) (end 30.05 14.9125) (width 0.25) (layer "F.Cu") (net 5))
 (segment (start 24.9 19.9) (end 23.5 18.5) (width 0.25) (layer "F.Cu") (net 5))
 (segment (start 23.5 18.5) (end 22.95 18.5) (width 0.25) (layer "F.Cu") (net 5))
 (segment (start 30.05 15.1) (end 31.15 16.2) (width 0.25) (layer "F.Cu") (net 5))
 (segment (start 27.55 19.9) (end 30.05 17.4) (width 0.25) (layer "F.Cu") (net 5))
 (via (at 21.7 17.25) (size 0.8) (drill 0.4) (layers "F.Cu" "B.Cu") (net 5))
 (via (at 31.15 16.2) (size 0.8) (drill 0.4) (layers "F.Cu" "B.Cu") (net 5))
 (segment (start 21.325 16.875) (end 21.7 17.25) (width 0.25) (layer "B.Cu") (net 5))
 (segment (start 31.15 16.2) (end 29.4 16.2) (width 0.25) (layer "B.Cu") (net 5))
 (segment (start 19.7375 16.875) (end 21.325 16.875) (width 0.25) (layer "B.Cu") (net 5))
 (segment (start 27.65 17.8) (end 26.125 17.8) (width 0.25) (layer "F.Cu") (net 2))
 (segment (start 26.125 17.8) (end 26.05 17.725) (width 0.25) (layer "F.Cu") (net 2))
 (via (at 27.65 17.8) (size 0.8) (drill 0.4) (layers "F.Cu" "B.Cu") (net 2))
 (segment (start 25.4625 17.525) (end 27.375 17.525) (width 0.25) (layer "B.Cu") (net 2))
 (segment (start 27.375 17.525) (end 27.65 17.8) (width 0.25) (layer "B.Cu") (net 2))
 (segment (start 25.4625 18.175) (end 26.775 18.175) (width 0.25) (layer "B.Cu") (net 18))
 (segment (start 27.15 18.55) (end 29.25 18.55) (width 0.25) (layer "B.Cu") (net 18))
 (segment (start 26.775 18.175) (end 27.15 18.55) (width 0.25) (layer "B.Cu") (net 18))
 (segment (start 29.25 18.55) (end 29.4 18.4) (width 0.25) (layer "B.Cu") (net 18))
 (segment (start 25.4625 18.825) (end 27.1875 20.55) (width 0.25) (layer "B.Cu") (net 19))
 (segment (start 27.1875 20.55) (end 29.4 20.55) (width 0.25) (layer "B.Cu") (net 19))
 (segment (start 20.625 20.963173) (end 22.211827 22.55) (width 0.25) (layer "F.Cu") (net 14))
 (segment (start 22.211827 22.55) (end 25.1 22.55) (width 0.25) (layer "F.Cu") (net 14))
 (segment (start 21.15 14.4) (end 20.625 14.925) (width 0.25) (layer "F.Cu") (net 14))
 (segment (start 20.625 15.45) (end 20.625 20.963173) (width 0.25) (layer "F.Cu") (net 14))
 (segment (start 20.625 14.925) (end 20.625 15.45) (width 0.25) (layer "F.Cu") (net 14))
 (via (at 25.1 22.55) (size 0.8) (drill 0.4) (layers "F.Cu" "B.Cu") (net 14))
 (via (at 21.15 14.4) (size 0.8) (drill 0.4) (layers "F.Cu" "B.Cu") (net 14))
 (segment (start 25.1 22.55) (end 23.9 21.35) (width 0.25) (layer "B.Cu") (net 14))
 (segment (start 23.9 21.35) (end 23.5 21.35) (width 0.25) (layer "B.Cu") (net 14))
 (segment (start 25.4625 12.975) (end 22.575 12.975) (width 0.25) (layer "B.Cu") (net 14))
 (segment (start 22.575 12.975) (end 21.15 14.4) (width 0.25) (layer "B.Cu") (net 14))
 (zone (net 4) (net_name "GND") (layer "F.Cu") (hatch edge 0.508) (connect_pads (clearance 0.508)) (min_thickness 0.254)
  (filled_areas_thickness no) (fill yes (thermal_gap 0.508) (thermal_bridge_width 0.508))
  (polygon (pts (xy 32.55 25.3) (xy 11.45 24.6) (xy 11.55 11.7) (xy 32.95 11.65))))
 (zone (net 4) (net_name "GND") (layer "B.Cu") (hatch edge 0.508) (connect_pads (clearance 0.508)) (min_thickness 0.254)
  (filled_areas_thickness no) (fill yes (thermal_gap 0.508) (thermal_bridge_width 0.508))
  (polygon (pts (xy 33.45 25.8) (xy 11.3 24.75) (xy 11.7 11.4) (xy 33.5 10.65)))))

